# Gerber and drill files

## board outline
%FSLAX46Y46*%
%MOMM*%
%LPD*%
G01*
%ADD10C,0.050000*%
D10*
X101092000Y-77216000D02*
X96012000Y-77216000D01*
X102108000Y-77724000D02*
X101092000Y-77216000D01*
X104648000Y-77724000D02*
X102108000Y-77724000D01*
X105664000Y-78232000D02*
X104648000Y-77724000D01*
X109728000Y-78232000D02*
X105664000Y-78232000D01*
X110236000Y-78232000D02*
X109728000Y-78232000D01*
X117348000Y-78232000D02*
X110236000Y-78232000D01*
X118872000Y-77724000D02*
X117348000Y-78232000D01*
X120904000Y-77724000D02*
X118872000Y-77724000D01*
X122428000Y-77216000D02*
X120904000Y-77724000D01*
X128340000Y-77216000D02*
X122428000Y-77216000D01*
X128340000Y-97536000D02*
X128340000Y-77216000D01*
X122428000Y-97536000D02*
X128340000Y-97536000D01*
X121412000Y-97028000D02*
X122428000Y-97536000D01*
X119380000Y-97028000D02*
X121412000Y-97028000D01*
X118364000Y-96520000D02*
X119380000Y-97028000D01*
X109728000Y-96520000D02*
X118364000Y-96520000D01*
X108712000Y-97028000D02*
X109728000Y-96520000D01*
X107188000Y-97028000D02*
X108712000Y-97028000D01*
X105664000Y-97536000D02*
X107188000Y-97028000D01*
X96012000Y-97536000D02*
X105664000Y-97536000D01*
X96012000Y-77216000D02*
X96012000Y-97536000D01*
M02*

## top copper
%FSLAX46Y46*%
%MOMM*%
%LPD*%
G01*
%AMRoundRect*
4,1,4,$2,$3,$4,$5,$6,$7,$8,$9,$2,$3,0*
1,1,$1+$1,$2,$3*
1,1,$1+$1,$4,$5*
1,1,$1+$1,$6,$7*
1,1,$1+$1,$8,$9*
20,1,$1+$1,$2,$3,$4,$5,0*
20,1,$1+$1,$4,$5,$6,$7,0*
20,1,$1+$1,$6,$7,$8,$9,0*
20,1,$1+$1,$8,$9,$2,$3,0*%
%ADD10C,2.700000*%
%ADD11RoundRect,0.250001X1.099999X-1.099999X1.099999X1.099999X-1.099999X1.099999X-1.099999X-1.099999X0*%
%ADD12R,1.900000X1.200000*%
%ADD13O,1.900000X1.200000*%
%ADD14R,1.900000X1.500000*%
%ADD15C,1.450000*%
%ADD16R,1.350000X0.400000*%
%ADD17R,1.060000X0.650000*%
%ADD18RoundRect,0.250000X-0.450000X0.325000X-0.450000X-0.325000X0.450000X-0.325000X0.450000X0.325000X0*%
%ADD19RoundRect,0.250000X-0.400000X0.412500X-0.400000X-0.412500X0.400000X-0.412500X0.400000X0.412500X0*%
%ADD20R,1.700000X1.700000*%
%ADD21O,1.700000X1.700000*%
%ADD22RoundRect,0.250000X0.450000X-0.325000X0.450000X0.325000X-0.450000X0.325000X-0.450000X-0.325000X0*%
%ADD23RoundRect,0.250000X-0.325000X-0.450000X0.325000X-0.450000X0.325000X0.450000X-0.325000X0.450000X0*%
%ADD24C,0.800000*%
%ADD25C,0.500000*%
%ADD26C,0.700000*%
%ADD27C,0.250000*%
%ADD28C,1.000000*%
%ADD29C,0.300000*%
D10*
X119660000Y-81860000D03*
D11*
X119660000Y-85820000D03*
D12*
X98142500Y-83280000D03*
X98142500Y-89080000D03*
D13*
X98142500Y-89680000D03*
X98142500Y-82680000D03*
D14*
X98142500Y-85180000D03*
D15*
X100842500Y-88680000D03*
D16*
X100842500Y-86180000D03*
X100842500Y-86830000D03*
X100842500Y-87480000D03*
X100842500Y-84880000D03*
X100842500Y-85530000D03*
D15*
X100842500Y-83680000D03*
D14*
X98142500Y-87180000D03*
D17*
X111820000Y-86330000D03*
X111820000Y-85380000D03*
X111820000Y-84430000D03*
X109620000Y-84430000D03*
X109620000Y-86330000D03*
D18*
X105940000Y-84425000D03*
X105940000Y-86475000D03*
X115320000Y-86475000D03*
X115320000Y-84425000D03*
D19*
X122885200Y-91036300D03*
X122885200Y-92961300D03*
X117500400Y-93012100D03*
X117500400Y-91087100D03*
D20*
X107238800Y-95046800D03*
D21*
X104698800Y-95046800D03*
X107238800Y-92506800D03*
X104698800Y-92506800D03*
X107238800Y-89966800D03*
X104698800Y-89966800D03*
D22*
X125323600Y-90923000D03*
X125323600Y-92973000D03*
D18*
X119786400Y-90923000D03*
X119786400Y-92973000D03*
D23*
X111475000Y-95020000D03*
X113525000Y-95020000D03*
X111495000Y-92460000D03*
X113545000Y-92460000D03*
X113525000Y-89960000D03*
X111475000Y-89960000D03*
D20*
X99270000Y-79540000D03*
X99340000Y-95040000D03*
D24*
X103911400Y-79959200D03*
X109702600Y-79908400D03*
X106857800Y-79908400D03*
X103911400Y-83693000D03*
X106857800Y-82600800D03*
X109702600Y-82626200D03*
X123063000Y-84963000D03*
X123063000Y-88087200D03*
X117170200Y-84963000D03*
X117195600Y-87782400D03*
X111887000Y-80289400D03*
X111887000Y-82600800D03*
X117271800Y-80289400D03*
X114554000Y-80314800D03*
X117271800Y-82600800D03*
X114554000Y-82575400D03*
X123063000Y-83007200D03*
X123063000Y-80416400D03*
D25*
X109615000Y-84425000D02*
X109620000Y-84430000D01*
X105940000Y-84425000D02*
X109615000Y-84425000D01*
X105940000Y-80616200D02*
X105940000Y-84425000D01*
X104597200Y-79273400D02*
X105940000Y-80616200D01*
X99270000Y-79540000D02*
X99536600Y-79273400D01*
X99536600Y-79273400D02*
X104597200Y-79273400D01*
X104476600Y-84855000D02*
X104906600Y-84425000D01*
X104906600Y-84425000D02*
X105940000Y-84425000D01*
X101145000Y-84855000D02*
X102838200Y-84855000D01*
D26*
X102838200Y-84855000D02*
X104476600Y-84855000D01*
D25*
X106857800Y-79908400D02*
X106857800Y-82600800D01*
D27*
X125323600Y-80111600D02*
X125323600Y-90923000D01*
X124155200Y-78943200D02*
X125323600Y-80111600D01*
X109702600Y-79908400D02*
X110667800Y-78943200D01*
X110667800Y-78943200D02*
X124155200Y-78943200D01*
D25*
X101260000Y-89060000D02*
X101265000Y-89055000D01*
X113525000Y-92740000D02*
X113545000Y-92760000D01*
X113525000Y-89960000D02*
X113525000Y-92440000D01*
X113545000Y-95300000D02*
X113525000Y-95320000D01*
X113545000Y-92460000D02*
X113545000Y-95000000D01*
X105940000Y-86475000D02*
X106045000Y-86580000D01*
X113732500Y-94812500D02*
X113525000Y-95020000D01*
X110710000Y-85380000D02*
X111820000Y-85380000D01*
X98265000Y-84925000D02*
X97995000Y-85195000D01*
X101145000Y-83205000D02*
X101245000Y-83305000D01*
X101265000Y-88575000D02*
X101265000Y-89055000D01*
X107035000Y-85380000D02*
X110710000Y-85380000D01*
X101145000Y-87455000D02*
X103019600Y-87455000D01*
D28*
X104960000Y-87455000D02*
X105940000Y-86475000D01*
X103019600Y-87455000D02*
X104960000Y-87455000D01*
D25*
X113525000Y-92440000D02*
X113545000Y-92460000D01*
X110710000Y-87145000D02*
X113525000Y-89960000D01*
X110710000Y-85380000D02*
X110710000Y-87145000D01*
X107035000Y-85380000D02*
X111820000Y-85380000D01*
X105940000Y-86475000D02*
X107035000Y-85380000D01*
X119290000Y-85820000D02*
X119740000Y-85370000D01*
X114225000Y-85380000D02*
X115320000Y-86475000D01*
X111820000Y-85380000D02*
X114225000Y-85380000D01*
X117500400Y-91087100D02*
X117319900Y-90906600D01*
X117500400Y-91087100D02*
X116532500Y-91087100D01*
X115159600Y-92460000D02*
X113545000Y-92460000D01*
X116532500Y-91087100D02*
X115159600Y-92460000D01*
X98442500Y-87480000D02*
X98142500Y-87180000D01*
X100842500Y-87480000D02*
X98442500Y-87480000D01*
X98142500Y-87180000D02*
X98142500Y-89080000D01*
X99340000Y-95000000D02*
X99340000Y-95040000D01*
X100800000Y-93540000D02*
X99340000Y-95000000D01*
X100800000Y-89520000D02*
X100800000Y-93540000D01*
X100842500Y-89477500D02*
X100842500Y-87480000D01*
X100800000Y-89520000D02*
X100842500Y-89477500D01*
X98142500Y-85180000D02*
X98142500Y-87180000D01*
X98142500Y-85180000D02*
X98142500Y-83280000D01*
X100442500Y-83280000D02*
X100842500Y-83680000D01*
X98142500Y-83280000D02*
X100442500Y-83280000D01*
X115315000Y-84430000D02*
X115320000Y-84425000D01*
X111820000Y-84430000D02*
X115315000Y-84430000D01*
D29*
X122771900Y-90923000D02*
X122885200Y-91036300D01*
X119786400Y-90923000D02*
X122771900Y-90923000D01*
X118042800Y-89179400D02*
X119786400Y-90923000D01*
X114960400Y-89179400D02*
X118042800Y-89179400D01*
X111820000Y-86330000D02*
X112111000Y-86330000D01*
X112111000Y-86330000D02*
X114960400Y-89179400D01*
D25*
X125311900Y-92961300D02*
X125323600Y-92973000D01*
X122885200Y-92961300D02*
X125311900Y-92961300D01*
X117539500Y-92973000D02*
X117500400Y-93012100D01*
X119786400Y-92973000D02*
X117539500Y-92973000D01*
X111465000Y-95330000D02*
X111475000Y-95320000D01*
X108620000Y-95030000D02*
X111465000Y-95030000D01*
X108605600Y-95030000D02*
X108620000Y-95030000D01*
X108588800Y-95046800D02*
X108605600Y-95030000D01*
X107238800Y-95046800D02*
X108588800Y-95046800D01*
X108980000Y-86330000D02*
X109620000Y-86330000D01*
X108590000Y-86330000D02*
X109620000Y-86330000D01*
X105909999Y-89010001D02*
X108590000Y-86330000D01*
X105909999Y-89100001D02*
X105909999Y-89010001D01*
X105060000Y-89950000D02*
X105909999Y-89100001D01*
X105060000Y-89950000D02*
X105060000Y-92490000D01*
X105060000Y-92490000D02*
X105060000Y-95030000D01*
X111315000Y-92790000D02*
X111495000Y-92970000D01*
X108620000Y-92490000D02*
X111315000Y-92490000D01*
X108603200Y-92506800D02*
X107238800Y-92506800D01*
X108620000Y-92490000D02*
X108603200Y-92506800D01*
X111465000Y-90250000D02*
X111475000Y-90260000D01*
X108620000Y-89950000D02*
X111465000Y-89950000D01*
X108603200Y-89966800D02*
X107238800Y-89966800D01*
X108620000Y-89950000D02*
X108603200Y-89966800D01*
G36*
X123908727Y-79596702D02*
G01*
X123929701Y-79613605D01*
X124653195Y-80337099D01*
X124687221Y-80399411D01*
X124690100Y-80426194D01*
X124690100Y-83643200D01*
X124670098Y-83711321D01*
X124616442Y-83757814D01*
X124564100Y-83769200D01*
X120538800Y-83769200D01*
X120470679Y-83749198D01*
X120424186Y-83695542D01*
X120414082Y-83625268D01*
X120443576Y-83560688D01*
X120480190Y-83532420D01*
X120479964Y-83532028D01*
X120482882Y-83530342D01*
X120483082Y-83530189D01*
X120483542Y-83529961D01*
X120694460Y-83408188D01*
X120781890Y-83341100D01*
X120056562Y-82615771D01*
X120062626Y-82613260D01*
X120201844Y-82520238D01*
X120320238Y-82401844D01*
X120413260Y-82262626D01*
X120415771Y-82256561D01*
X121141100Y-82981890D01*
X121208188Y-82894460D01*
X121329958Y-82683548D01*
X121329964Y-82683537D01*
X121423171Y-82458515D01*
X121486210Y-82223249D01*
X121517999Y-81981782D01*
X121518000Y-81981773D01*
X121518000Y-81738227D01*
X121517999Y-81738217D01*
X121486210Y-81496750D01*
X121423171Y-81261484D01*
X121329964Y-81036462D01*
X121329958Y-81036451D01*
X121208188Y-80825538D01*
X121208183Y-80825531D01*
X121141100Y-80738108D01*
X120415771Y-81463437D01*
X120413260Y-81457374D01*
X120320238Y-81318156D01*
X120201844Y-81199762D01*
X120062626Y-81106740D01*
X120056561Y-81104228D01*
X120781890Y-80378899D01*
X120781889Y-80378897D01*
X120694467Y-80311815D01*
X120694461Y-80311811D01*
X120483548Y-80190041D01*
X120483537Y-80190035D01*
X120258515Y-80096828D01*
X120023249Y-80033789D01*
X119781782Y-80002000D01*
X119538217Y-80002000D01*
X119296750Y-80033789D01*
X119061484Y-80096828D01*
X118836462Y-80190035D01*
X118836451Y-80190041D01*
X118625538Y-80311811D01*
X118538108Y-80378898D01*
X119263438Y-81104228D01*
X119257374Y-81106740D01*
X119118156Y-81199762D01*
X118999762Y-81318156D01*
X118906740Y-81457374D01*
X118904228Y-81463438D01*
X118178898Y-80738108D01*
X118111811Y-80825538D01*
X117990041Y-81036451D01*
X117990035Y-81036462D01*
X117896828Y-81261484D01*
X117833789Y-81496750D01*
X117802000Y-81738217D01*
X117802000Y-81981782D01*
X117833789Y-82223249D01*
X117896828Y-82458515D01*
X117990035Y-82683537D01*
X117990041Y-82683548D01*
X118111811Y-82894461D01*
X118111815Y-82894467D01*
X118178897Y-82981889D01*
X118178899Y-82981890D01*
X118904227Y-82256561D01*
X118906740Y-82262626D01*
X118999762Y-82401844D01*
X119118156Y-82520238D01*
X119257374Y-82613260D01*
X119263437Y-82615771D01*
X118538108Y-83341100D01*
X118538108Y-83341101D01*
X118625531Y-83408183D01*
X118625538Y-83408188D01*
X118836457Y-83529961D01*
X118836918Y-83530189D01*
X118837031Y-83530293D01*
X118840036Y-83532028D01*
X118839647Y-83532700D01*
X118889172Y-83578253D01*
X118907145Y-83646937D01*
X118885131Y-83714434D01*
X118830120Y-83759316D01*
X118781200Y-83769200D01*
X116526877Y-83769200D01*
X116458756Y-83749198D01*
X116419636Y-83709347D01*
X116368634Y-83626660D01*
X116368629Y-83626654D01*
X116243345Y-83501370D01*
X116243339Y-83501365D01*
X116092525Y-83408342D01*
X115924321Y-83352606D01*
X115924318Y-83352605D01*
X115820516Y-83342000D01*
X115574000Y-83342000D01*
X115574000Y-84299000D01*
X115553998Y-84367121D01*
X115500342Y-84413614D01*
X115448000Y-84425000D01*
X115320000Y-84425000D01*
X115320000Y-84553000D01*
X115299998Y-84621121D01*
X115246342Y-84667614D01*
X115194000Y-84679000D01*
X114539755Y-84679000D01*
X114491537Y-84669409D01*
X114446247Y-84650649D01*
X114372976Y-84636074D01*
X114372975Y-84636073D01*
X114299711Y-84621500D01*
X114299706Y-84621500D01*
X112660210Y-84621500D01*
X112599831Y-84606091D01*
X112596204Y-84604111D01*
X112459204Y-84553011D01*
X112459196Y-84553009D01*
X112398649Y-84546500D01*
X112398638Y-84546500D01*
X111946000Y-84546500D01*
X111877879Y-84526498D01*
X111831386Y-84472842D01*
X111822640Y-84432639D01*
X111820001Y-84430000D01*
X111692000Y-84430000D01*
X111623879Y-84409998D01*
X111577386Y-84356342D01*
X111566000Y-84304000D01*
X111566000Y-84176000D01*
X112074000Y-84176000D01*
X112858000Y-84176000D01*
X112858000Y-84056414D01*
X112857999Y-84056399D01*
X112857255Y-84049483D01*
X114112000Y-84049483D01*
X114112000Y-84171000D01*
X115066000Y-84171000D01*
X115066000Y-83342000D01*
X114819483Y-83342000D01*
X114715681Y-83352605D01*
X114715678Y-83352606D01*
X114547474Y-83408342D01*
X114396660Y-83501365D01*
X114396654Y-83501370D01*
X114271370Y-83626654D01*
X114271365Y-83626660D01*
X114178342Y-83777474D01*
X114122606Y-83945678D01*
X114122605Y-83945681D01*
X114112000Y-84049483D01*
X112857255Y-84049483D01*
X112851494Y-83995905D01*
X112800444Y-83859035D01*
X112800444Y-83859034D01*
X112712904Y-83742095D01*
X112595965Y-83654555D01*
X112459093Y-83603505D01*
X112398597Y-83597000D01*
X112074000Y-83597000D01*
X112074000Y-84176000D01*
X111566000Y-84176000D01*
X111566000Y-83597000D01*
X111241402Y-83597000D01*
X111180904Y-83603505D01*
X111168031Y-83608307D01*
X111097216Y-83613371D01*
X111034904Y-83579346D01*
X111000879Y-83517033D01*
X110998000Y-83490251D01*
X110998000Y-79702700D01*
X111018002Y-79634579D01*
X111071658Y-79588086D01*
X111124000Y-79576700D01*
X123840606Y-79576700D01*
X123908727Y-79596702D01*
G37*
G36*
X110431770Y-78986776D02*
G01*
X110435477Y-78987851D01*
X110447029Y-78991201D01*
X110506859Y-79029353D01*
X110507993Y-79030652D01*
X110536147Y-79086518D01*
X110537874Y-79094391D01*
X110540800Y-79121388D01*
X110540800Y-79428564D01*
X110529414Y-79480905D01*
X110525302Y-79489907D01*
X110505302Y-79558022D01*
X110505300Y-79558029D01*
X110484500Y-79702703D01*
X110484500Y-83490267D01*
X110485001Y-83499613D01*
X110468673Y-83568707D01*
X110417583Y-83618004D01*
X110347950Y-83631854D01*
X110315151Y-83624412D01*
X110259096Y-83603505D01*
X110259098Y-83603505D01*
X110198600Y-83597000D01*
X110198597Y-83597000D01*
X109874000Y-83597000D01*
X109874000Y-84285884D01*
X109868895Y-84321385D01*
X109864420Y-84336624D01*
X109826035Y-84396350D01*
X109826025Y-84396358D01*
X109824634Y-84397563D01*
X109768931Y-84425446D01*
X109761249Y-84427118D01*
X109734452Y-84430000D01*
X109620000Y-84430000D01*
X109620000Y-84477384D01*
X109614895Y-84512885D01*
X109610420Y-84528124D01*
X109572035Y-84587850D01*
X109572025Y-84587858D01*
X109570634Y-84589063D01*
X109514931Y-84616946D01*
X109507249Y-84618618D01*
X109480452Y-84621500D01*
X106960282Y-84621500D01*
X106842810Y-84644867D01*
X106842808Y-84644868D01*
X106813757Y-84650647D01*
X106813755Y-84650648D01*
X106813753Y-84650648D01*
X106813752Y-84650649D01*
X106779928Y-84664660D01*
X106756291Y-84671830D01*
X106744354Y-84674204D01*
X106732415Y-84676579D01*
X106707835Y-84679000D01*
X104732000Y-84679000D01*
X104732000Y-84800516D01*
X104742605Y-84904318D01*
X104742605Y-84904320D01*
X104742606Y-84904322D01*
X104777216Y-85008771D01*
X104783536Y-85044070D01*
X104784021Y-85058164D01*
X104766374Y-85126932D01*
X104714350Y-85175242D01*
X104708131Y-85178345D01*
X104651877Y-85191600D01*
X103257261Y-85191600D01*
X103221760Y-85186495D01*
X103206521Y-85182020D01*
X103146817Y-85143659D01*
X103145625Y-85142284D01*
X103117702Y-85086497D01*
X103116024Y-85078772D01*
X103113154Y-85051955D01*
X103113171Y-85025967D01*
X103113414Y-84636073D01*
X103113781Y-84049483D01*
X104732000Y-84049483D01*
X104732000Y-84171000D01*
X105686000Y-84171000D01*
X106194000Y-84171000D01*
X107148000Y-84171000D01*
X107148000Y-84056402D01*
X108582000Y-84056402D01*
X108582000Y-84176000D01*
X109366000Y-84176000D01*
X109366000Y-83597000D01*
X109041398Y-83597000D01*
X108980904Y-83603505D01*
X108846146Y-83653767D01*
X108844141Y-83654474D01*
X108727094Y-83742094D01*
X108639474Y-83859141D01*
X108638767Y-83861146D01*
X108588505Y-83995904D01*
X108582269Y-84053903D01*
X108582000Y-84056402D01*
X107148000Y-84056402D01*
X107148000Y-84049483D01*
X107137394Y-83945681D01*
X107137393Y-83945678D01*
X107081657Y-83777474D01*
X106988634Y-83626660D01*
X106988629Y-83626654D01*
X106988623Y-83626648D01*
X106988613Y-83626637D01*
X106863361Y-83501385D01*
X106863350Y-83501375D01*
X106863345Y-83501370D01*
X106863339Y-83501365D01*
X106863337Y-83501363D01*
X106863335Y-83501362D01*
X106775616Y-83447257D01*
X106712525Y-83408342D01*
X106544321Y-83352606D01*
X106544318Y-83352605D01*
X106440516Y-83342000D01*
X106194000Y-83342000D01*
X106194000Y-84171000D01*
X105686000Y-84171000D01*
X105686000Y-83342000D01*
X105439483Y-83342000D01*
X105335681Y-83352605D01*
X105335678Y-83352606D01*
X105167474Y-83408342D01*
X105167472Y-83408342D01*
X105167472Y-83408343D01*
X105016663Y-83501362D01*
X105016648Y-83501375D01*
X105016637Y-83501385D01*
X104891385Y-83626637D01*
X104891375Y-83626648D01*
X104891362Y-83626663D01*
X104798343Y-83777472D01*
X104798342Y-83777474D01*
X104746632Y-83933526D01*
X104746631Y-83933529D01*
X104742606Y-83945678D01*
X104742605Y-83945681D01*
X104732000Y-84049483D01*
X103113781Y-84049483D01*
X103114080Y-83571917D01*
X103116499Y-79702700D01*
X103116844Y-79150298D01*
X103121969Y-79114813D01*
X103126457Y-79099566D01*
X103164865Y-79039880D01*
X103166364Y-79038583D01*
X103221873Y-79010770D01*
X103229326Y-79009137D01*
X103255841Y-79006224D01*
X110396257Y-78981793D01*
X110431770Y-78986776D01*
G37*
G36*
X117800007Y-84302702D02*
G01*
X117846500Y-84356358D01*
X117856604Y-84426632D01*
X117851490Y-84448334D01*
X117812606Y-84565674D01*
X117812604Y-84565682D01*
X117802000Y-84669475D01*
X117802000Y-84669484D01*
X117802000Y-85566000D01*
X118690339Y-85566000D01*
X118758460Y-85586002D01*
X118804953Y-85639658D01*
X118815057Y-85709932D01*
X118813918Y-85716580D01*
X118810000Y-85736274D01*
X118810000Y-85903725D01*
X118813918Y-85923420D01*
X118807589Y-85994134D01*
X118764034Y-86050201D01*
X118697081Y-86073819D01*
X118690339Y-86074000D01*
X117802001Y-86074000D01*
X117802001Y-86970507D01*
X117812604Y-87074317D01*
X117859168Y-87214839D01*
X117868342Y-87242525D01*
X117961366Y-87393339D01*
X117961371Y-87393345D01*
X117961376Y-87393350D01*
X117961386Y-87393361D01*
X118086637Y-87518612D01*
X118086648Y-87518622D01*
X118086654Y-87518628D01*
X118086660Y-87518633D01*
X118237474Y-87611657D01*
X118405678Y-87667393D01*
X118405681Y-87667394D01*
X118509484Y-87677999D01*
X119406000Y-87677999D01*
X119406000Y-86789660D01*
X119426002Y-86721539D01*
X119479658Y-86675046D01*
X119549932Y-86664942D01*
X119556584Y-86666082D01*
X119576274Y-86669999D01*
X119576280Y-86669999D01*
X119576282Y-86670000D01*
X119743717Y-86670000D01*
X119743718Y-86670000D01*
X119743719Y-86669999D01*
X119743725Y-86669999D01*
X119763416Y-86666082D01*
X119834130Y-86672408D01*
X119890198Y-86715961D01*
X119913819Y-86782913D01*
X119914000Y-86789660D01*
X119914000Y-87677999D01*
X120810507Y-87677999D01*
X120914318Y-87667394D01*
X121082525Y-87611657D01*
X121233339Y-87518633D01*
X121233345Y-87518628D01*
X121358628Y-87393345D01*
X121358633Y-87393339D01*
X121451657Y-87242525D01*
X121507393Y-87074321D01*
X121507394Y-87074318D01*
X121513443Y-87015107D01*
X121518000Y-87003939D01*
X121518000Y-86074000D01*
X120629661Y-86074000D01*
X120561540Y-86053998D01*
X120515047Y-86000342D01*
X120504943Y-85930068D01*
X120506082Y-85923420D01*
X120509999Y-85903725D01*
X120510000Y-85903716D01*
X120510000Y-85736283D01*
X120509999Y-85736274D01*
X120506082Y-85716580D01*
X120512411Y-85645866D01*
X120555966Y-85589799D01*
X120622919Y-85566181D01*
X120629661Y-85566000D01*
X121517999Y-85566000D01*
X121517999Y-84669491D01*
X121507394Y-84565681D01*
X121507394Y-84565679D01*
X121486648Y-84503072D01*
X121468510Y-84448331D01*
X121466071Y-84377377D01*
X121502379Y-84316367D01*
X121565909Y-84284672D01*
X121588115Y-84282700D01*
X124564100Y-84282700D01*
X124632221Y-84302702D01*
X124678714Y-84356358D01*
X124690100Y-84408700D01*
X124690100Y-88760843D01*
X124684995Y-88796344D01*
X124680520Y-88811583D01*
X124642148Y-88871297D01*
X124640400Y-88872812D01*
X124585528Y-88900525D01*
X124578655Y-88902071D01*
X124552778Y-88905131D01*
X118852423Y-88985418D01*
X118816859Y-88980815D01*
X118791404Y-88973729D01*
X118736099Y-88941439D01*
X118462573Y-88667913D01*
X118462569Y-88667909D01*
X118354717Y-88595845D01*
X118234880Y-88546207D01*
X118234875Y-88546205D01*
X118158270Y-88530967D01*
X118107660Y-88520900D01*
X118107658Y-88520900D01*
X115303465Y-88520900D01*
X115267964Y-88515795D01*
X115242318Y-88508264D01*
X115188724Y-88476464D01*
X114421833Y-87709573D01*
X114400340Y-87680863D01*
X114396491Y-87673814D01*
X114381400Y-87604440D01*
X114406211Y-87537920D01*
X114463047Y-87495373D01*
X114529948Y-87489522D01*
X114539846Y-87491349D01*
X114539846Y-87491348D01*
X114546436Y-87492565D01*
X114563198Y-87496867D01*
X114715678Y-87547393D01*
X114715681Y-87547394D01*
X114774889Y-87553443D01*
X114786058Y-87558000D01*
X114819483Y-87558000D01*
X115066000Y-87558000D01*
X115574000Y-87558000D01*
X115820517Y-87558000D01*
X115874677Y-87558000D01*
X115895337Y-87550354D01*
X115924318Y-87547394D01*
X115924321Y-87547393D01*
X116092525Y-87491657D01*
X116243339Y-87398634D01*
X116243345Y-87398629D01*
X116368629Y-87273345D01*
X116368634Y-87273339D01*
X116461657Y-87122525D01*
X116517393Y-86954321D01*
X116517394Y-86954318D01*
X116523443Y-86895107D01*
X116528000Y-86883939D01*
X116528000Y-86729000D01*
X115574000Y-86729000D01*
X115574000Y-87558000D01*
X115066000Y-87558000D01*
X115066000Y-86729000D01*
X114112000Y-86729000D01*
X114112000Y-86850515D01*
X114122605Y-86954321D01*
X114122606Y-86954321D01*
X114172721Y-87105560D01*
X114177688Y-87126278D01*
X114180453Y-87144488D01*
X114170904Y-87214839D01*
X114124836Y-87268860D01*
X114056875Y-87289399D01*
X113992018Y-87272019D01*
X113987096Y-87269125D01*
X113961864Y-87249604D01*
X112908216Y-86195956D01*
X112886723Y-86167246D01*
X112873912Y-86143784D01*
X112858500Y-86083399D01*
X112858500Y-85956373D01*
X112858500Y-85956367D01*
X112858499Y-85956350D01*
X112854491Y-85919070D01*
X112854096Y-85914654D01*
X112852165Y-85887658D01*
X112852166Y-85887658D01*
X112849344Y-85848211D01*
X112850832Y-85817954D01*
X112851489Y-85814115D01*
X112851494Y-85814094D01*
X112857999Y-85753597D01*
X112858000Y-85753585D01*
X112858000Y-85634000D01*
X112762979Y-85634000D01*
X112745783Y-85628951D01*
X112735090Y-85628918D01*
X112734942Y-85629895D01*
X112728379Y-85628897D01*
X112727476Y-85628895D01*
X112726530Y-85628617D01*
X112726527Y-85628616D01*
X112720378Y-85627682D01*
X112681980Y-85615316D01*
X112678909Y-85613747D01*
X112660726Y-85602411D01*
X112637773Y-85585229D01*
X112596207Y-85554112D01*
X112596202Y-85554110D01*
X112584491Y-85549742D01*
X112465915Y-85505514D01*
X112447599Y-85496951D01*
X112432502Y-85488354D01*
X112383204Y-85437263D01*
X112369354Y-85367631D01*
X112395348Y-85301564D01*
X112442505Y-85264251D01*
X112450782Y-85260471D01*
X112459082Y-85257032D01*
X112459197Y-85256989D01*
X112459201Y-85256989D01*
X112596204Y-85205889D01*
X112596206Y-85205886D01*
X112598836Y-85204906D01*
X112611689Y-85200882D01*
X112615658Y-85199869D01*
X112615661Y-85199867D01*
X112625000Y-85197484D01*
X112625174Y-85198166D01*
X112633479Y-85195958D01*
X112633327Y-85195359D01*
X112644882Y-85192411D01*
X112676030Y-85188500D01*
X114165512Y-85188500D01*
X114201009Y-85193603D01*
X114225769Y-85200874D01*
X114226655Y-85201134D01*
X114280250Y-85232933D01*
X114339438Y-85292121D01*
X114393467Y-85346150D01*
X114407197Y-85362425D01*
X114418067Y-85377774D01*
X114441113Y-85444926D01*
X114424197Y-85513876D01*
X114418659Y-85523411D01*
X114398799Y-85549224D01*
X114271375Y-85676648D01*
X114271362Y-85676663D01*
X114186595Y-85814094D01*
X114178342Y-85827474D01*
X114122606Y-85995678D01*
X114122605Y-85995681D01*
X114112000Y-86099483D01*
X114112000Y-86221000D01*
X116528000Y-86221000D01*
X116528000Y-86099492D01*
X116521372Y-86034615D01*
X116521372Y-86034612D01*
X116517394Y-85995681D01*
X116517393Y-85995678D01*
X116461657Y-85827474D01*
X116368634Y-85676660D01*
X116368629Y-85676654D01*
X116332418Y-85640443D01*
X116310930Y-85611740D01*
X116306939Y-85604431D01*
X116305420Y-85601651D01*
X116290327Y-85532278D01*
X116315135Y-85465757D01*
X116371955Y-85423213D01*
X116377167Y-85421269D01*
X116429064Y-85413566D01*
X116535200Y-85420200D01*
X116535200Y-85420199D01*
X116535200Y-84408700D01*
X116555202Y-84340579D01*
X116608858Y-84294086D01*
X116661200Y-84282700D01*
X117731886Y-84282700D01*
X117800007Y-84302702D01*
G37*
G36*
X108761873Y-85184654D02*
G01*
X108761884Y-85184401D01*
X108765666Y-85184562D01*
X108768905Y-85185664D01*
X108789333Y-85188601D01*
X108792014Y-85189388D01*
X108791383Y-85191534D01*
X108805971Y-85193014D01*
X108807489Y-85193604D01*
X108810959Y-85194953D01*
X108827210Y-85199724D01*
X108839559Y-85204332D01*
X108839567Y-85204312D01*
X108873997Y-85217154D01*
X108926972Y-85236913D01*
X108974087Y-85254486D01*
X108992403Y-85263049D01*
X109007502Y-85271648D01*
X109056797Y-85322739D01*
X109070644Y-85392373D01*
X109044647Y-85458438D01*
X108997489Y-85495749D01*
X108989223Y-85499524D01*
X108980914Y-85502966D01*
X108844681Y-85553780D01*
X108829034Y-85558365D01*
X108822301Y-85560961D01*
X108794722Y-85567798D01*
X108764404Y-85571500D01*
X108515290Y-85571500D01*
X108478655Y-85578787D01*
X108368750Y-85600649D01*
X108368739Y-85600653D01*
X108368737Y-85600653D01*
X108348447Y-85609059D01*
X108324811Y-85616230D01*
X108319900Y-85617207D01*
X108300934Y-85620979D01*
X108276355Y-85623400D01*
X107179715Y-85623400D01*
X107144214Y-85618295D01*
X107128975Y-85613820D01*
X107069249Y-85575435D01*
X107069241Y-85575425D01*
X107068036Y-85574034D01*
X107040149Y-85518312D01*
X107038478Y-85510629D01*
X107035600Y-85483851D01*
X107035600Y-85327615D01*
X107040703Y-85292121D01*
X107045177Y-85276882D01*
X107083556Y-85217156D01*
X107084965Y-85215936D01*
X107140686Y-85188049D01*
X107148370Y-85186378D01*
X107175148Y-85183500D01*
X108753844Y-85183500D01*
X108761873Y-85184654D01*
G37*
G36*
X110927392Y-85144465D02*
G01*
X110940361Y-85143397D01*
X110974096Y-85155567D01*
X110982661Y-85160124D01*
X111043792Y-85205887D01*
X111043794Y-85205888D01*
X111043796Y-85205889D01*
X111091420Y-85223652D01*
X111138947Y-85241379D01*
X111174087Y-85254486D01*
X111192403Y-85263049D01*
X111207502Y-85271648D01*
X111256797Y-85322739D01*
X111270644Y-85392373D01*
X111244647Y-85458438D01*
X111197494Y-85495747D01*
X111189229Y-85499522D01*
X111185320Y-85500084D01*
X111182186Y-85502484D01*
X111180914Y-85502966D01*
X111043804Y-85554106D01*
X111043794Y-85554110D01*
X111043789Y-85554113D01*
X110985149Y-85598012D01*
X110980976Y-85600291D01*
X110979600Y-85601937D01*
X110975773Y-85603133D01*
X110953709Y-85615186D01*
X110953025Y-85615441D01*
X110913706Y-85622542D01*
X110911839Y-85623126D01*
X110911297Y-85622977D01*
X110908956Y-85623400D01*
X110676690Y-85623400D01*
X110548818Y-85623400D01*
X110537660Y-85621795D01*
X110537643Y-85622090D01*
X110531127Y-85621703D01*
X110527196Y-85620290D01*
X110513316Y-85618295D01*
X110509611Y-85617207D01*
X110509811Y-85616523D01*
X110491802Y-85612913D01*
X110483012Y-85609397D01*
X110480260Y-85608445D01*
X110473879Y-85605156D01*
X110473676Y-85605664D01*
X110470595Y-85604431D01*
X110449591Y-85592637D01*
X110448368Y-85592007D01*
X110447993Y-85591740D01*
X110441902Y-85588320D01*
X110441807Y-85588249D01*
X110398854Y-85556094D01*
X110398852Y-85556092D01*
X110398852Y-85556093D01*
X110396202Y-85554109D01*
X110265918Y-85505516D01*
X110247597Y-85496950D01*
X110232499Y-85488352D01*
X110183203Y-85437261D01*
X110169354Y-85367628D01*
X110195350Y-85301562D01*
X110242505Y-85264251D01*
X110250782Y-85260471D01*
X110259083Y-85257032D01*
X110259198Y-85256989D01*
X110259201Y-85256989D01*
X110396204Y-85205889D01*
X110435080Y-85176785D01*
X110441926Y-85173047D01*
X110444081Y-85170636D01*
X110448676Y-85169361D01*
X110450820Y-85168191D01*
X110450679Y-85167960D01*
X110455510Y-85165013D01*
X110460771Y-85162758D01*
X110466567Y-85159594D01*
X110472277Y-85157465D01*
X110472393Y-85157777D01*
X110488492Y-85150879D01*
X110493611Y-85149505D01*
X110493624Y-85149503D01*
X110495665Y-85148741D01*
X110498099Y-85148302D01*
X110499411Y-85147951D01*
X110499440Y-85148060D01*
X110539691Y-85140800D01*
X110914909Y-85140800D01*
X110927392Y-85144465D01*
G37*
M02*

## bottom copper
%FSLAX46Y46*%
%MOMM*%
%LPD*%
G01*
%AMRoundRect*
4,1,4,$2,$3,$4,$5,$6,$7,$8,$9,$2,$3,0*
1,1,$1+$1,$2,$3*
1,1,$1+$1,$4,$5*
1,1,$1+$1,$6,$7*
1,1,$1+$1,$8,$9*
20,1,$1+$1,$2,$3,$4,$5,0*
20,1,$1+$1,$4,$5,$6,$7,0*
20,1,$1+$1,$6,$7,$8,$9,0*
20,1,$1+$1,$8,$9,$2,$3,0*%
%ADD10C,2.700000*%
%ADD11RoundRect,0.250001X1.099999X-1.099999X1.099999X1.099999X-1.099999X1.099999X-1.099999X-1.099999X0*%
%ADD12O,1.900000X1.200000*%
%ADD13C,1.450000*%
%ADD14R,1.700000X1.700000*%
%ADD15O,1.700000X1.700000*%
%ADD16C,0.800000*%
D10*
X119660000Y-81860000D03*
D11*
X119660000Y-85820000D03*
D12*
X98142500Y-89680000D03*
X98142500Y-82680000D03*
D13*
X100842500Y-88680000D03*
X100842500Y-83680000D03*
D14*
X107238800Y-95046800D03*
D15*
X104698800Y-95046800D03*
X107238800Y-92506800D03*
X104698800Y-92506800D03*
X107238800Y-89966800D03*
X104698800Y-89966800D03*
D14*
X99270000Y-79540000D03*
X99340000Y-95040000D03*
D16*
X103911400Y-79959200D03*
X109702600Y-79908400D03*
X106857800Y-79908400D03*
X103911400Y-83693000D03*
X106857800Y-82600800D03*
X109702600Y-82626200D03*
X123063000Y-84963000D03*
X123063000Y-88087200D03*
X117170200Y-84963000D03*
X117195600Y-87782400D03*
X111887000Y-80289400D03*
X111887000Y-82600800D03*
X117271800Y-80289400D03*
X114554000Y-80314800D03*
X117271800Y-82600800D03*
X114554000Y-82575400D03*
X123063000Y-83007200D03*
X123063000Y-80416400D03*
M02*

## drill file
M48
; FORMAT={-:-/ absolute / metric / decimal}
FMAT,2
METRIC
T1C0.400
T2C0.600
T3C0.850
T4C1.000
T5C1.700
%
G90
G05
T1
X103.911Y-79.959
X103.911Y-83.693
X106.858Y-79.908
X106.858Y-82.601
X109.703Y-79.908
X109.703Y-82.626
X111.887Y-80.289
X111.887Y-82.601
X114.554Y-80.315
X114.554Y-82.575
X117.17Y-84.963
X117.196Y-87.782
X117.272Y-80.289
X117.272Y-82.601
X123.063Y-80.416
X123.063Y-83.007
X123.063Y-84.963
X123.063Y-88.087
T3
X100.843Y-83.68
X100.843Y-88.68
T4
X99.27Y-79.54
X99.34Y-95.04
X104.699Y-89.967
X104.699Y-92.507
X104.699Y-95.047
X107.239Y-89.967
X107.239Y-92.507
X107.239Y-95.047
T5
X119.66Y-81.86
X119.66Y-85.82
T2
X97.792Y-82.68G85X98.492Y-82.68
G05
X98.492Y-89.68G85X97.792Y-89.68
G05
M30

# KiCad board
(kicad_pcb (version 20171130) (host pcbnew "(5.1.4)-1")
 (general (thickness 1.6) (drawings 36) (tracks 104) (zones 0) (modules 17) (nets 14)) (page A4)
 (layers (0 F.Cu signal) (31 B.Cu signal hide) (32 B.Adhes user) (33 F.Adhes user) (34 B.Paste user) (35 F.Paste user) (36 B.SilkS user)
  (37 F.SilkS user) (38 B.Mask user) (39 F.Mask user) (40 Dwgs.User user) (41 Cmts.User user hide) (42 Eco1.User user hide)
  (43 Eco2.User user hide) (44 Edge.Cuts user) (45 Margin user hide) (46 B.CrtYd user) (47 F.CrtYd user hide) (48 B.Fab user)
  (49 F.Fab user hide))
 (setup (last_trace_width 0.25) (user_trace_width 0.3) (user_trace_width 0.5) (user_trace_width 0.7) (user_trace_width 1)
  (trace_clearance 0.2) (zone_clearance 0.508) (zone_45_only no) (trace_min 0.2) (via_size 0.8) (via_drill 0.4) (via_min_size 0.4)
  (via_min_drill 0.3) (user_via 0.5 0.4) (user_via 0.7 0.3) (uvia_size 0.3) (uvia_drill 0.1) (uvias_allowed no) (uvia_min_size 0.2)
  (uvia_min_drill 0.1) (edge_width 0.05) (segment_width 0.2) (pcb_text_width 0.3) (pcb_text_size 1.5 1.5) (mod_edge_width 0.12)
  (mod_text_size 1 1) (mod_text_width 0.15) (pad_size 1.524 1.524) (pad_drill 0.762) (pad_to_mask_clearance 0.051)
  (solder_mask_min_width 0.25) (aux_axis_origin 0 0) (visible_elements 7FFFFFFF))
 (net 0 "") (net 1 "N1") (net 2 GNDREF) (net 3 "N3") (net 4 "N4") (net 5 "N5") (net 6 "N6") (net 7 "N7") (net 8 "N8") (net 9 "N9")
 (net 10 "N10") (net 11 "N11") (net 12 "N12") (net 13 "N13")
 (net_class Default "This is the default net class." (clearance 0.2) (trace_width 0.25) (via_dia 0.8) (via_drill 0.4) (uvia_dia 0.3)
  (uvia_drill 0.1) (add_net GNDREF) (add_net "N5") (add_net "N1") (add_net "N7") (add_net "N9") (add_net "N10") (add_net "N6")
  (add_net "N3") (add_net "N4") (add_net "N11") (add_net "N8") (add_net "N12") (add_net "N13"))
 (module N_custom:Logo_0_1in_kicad (layer F.Cu) (at 108.3 81.51)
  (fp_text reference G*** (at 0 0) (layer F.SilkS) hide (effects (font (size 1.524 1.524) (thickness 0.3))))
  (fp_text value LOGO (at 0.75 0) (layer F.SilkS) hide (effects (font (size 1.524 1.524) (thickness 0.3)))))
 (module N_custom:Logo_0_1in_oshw (layer F.Cu) (at 115.92 81.36)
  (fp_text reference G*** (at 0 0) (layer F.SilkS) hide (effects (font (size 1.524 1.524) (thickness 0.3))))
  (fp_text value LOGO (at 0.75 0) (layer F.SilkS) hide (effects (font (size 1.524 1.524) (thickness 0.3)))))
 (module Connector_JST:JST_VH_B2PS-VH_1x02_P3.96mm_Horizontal (layer F.Cu) (at 119.66 85.82 90)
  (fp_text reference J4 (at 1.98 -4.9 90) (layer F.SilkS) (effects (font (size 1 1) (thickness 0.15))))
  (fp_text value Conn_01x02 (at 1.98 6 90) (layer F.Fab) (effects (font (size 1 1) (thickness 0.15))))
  (pad 2 thru_hole circle (at 3.96 0 90) (size 2.7 2.7) (drill 1.7) (layers *.Cu *.Mask) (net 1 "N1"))
  (pad 1 thru_hole roundrect (at 0 0 90) (size 2.7 2.7) (drill 1.7) (layers *.Cu *.Mask) (roundrect_rratio 0.09259299999999999)
   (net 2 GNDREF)))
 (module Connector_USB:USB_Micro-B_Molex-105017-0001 (layer F.Cu) (at 99.38 86.18 270)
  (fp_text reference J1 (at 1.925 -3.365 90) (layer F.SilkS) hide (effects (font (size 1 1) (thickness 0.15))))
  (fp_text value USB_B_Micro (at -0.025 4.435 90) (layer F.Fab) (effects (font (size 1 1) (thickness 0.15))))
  (pad 6 smd rect (at -2.9 1.2375 270) (size 1.2 1.9) (layers F.Cu F.Mask) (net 2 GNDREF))
  (pad 6 smd rect (at 2.9 1.2375 270) (size 1.2 1.9) (layers F.Cu F.Mask) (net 2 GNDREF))
  (pad 6 thru_hole oval (at 3.5 1.2375 270) (size 1.2 1.9) (drill oval 0.6 1.3) (layers *.Cu *.Mask) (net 2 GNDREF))
  (pad 6 thru_hole oval (at -3.5 1.2375 90) (size 1.2 1.9) (drill oval 0.6 1.3) (layers *.Cu *.Mask) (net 2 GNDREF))
  (pad 6 smd rect (at -1 1.2375 270) (size 1.5 1.9) (layers F.Cu F.Paste F.Mask) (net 2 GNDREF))
  (pad 6 thru_hole circle (at 2.5 -1.4625 270) (size 1.45 1.45) (drill 0.85) (layers *.Cu *.Mask) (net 2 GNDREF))
  (pad 3 smd rect (at 0 -1.4625 270) (size 0.4 1.35) (layers F.Cu F.Paste F.Mask) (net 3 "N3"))
  (pad 4 smd rect (at 0.65 -1.4625 270) (size 0.4 1.35) (layers F.Cu F.Paste F.Mask) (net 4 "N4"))
  (pad 5 smd rect (at 1.3 -1.4625 270) (size 0.4 1.35) (layers F.Cu F.Paste F.Mask) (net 2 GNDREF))
  (pad 1 smd rect (at -1.3 -1.4625 270) (size 0.4 1.35) (layers F.Cu F.Paste F.Mask) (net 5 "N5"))
  (pad 2 smd rect (at -0.65 -1.4625 270) (size 0.4 1.35) (layers F.Cu F.Paste F.Mask) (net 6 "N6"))
  (pad 6 thru_hole circle (at -2.5 -1.4625 270) (size 1.45 1.45) (drill 0.85) (layers *.Cu *.Mask) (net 2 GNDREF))
  (pad 6 smd rect (at 1 1.2375 270) (size 1.5 1.9) (layers F.Cu F.Paste F.Mask) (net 2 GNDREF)))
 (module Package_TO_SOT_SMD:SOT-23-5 (layer F.Cu) (at 110.72 85.38 180)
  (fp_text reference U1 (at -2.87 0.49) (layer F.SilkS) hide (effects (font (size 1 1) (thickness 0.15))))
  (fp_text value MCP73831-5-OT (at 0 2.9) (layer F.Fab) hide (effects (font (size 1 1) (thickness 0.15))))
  (pad 1 smd rect (at -1.1 -0.95 180) (size 1.06 0.65) (layers F.Cu F.Paste F.Mask) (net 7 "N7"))
  (pad 2 smd rect (at -1.1 0 180) (size 1.06 0.65) (layers F.Cu F.Paste F.Mask) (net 2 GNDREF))
  (pad 3 smd rect (at -1.1 0.95 180) (size 1.06 0.65) (layers F.Cu F.Paste F.Mask) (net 1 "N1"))
  (pad 4 smd rect (at 1.1 0.95 180) (size 1.06 0.65) (layers F.Cu F.Paste F.Mask) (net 5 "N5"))
  (pad 5 smd rect (at 1.1 -0.95 180) (size 1.06 0.65) (layers F.Cu F.Paste F.Mask) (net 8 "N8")))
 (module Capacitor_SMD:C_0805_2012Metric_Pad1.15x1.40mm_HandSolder (layer F.Cu) (at 105.94 85.45 270)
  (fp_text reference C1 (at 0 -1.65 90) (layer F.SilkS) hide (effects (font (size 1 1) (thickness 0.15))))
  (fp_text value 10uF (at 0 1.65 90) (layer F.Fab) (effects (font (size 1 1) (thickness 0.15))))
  (pad 1 smd roundrect (at -1.025 0 270) (size 1.15 1.4) (layers F.Cu F.Paste F.Mask) (roundrect_rratio 0.217391) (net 5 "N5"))
  (pad 2 smd roundrect (at 1.025 0 270) (size 1.15 1.4) (layers F.Cu F.Paste F.Mask) (roundrect_rratio 0.217391) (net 2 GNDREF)))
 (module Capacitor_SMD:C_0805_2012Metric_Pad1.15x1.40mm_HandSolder (layer F.Cu) (at 115.32 85.45 270)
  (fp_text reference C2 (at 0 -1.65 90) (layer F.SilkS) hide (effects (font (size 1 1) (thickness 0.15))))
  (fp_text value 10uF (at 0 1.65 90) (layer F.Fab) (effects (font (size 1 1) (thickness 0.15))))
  (pad 2 smd roundrect (at 1.025 0 270) (size 1.15 1.4) (layers F.Cu F.Paste F.Mask) (roundrect_rratio 0.217391) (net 2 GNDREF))
  (pad 1 smd roundrect (at -1.025 0 270) (size 1.15 1.4) (layers F.Cu F.Paste F.Mask) (roundrect_rratio 0.217391) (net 1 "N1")))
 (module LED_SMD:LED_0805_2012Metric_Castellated (layer F.Cu) (at 122.8852 91.9988 270)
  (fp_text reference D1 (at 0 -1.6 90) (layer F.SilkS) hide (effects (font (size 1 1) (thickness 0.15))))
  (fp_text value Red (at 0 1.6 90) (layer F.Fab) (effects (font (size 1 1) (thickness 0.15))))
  (pad 1 smd roundrect (at -0.9625 0 270) (size 1.325 1.3) (layers F.Cu F.Paste F.Mask) (roundrect_rratio 0.192308) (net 7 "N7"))
  (pad 2 smd roundrect (at 0.9625 0 270) (size 1.325 1.3) (layers F.Cu F.Paste F.Mask) (roundrect_rratio 0.192308) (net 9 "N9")))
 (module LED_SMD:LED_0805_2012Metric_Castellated (layer F.Cu) (at 117.5004 92.0496 270)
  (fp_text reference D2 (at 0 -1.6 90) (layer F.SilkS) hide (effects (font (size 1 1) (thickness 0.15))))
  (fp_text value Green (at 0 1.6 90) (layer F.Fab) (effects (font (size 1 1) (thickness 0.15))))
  (pad 2 smd roundrect (at 0.9625 0 270) (size 1.325 1.3) (layers F.Cu F.Paste F.Mask) (roundrect_rratio 0.192308) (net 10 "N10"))
  (pad 1 smd roundrect (at -0.9625 0 270) (size 1.325 1.3) (layers F.Cu F.Paste F.Mask) (roundrect_rratio 0.192308) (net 2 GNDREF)))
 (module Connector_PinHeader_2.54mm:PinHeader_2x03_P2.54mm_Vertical (layer F.Cu) (at 107.2388 95.0468 180)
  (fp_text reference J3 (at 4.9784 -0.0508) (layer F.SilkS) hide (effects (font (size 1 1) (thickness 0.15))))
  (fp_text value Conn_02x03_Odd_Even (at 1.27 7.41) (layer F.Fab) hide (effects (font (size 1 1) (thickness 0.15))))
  (pad 1 thru_hole rect (at 0 0 180) (size 1.7 1.7) (drill 1) (layers *.Cu *.Mask) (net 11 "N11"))
  (pad 2 thru_hole oval (at 2.54 0 180) (size 1.7 1.7) (drill 1) (layers *.Cu *.Mask) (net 8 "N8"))
  (pad 3 thru_hole oval (at 0 2.54 180) (size 1.7 1.7) (drill 1) (layers *.Cu *.Mask) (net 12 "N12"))
  (pad 4 thru_hole oval (at 2.54 2.54 180) (size 1.7 1.7) (drill 1) (layers *.Cu *.Mask) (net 8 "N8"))
  (pad 5 thru_hole oval (at 0 5.08 180) (size 1.7 1.7) (drill 1) (layers *.Cu *.Mask) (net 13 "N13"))
  (pad 6 thru_hole oval (at 2.54 5.08 180) (size 1.7 1.7) (drill 1) (layers *.Cu *.Mask) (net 8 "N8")))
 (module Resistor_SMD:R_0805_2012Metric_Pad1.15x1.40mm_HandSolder (layer F.Cu) (at 125.3236 91.948 90)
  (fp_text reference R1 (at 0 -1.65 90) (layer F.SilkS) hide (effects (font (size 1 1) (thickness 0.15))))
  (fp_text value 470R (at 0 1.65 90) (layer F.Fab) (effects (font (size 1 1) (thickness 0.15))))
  (pad 2 smd roundrect (at 1.025 0 90) (size 1.15 1.4) (layers F.Cu F.Paste F.Mask) (roundrect_rratio 0.217391) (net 5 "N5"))
  (pad 1 smd roundrect (at -1.025 0 90) (size 1.15 1.4) (layers F.Cu F.Paste F.Mask) (roundrect_rratio 0.217391) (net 9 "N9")))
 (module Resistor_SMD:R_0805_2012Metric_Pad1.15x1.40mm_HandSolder (layer F.Cu) (at 119.7864 91.948 270)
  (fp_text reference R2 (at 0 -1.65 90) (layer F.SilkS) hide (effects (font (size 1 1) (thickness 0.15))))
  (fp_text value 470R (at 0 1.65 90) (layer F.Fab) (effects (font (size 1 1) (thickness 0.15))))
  (pad 1 smd roundrect (at -1.025 0 270) (size 1.15 1.4) (layers F.Cu F.Paste F.Mask) (roundrect_rratio 0.217391) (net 7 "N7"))
  (pad 2 smd roundrect (at 1.025 0 270) (size 1.15 1.4) (layers F.Cu F.Paste F.Mask) (roundrect_rratio 0.217391) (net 10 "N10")))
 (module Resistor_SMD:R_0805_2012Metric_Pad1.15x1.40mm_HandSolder (layer F.Cu) (at 112.5 95.02)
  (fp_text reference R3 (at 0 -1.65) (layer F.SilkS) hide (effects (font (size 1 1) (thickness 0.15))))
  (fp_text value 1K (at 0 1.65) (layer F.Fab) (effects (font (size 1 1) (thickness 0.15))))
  (pad 1 smd roundrect (at -1.025 0) (size 1.15 1.4) (layers F.Cu F.Paste F.Mask) (roundrect_rratio 0.217391) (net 11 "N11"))
  (pad 2 smd roundrect (at 1.025 0) (size 1.15 1.4) (layers F.Cu F.Paste F.Mask) (roundrect_rratio 0.217391) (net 2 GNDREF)))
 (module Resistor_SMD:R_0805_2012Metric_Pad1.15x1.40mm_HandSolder (layer F.Cu) (at 112.52 92.46)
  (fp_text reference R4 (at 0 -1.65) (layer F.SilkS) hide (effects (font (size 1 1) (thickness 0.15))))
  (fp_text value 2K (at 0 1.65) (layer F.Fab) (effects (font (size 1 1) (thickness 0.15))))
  (pad 1 smd roundrect (at -1.025 0) (size 1.15 1.4) (layers F.Cu F.Paste F.Mask) (roundrect_rratio 0.217391) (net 12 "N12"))
  (pad 2 smd roundrect (at 1.025 0) (size 1.15 1.4) (layers F.Cu F.Paste F.Mask) (roundrect_rratio 0.217391) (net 2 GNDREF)))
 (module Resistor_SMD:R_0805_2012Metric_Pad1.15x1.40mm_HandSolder (layer F.Cu) (at 112.5 89.96)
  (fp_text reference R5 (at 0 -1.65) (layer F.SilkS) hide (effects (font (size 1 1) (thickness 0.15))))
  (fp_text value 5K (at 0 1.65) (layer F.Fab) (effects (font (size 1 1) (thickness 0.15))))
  (pad 2 smd roundrect (at 1.025 0) (size 1.15 1.4) (layers F.Cu F.Paste F.Mask) (roundrect_rratio 0.217391) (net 2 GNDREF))
  (pad 1 smd roundrect (at -1.025 0) (size 1.15 1.4) (layers F.Cu F.Paste F.Mask) (roundrect_rratio 0.217391) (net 13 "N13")))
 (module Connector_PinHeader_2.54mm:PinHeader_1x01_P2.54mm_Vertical (layer F.Cu) (at 99.27 79.54)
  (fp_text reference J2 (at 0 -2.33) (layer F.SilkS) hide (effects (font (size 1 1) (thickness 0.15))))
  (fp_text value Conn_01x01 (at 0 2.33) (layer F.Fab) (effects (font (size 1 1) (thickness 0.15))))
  (pad 1 thru_hole rect (at 0 0) (size 1.7 1.7) (drill 1) (layers *.Cu *.Mask) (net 5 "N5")))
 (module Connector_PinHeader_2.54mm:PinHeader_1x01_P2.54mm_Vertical (layer F.Cu) (at 99.34 95.04)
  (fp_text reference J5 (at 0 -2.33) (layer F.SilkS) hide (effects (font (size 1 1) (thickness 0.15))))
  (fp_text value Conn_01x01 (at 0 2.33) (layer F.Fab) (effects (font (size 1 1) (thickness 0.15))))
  (pad 1 thru_hole rect (at 0 0) (size 1.7 1.7) (drill 1) (layers *.Cu *.Mask) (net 2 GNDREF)))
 (gr_line (start 101.092 77.216) (end 96.012 77.216) (layer Edge.Cuts) (width 0.05))
 (gr_line (start 102.108 77.724) (end 101.092 77.216) (layer Edge.Cuts) (width 0.05))
 (gr_line (start 104.648 77.724) (end 102.108 77.724) (layer Edge.Cuts) (width 0.05))
 (gr_line (start 105.664 78.232) (end 104.648 77.724) (layer Edge.Cuts) (width 0.05))
 (gr_line (start 109.728 78.232) (end 105.664 78.232) (layer Edge.Cuts) (width 0.05))
 (gr_line (start 110.236 78.232) (end 109.728 78.232) (layer Edge.Cuts) (width 0.05))
 (gr_line (start 117.348 78.232) (end 110.236 78.232) (layer Edge.Cuts) (width 0.05))
 (gr_line (start 118.872 77.724) (end 117.348 78.232) (layer Edge.Cuts) (width 0.05))
 (gr_line (start 120.904 77.724) (end 118.872 77.724) (layer Edge.Cuts) (width 0.05))
 (gr_line (start 122.428 77.216) (end 120.904 77.724) (layer Edge.Cuts) (width 0.05))
 (gr_line (start 128.34 77.216) (end 122.428 77.216) (layer Edge.Cuts) (width 0.05))
 (gr_line (start 128.34 97.536) (end 128.34 77.216) (layer Edge.Cuts) (width 0.05))
 (gr_line (start 122.428 97.536) (end 128.34 97.536) (layer Edge.Cuts) (width 0.05))
 (gr_line (start 121.412 97.028) (end 122.428 97.536) (layer Edge.Cuts) (width 0.05))
 (gr_line (start 119.38 97.028) (end 121.412 97.028) (layer Edge.Cuts) (width 0.05))
 (gr_line (start 118.364 96.52) (end 119.38 97.028) (layer Edge.Cuts) (width 0.05))
 (gr_line (start 109.728 96.52) (end 118.364 96.52) (layer Edge.Cuts) (width 0.05))
 (gr_line (start 108.712 97.028) (end 109.728 96.52) (layer Edge.Cuts) (width 0.05))
 (gr_line (start 107.188 97.028) (end 108.712 97.028) (layer Edge.Cuts) (width 0.05))
 (gr_line (start 105.664 97.536) (end 107.188 97.028) (layer Edge.Cuts) (width 0.05))
 (gr_line (start 96.012 97.536) (end 105.664 97.536) (layer Edge.Cuts) (width 0.05))
 (gr_line (start 96.012 77.216) (end 96.012 97.536) (layer Edge.Cuts) (width 0.05))
 (segment (start 109.615 84.425) (end 109.62 84.43) (width 0.5) (layer F.Cu) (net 5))
 (segment (start 105.94 84.425) (end 109.615 84.425) (width 0.5) (layer F.Cu) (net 5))
 (segment (start 105.94 80.6162) (end 105.94 84.425) (width 0.5) (layer F.Cu) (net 5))
 (segment (start 104.5972 79.2734) (end 105.94 80.6162) (width 0.5) (layer F.Cu) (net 5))
 (segment (start 99.27 79.54) (end 99.5366 79.2734) (width 0.5) (layer F.Cu) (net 5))
 (segment (start 99.5366 79.2734) (end 104.5972 79.2734) (width 0.5) (layer F.Cu) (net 5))
 (segment (start 104.4766 84.855) (end 104.9066 84.425) (width 0.5) (layer F.Cu) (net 5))
 (segment (start 104.9066 84.425) (end 105.94 84.425) (width 0.5) (layer F.Cu) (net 5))
 (segment (start 101.145 84.855) (end 102.8382 84.855) (width 0.5) (layer F.Cu) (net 5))
 (segment (start 102.8382 84.855) (end 104.4766 84.855) (width 0.7) (layer F.Cu) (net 5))
 (via (at 103.9114 79.9592) (size 0.8) (drill 0.4) (layers F.Cu B.Cu) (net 5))
 (via (at 109.7026 79.9084) (size 0.8) (drill 0.4) (layers F.Cu B.Cu) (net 5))
 (via (at 106.8578 79.9084) (size 0.8) (drill 0.4) (layers F.Cu B.Cu) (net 5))
 (via (at 103.9114 83.693) (size 0.8) (drill 0.4) (layers F.Cu B.Cu) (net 5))
 (via (at 106.8578 82.6008) (size 0.8) (drill 0.4) (layers F.Cu B.Cu) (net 5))
 (segment (start 106.8578 79.9084) (end 106.8578 82.6008) (width 0.5) (layer F.Cu) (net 5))
 (via (at 109.7026 82.6262) (size 0.8) (drill 0.4) (layers F.Cu B.Cu) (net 5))
 (segment (start 125.3236 80.1116) (end 125.3236 90.923) (width 0.25) (layer F.Cu) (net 5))
 (segment (start 124.1552 78.9432) (end 125.3236 80.1116) (width 0.25) (layer F.Cu) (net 5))
 (segment (start 109.7026 79.9084) (end 110.6678 78.9432) (width 0.25) (layer F.Cu) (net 5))
 (segment (start 110.6678 78.9432) (end 124.1552 78.9432) (width 0.25) (layer F.Cu) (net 5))
 (segment (start 101.26 89.06) (end 101.265 89.055) (width 0.5) (layer F.Cu) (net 2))
 (segment (start 113.525 92.74) (end 113.545 92.76) (width 0.5) (layer F.Cu) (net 2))
 (segment (start 113.525 89.96) (end 113.525 92.44) (width 0.5) (layer F.Cu) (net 2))
 (segment (start 113.545 95.3) (end 113.525 95.32) (width 0.5) (layer F.Cu) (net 2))
 (segment (start 113.545 92.46) (end 113.545 95) (width 0.5) (layer F.Cu) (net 2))
 (segment (start 105.94 86.475) (end 106.045 86.58) (width 0.5) (layer F.Cu) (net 2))
 (segment (start 113.7325 94.8125) (end 113.525 95.02) (width 0.5) (layer F.Cu) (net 2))
 (segment (start 110.71 85.38) (end 111.82 85.38) (width 0.5) (layer F.Cu) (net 2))
 (segment (start 98.265 84.925) (end 97.995 85.195) (width 0.5) (layer F.Cu) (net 2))
 (segment (start 101.145 83.205) (end 101.245 83.305) (width 0.5) (layer F.Cu) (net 2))
 (segment (start 101.265 88.575) (end 101.265 89.055) (width 0.5) (layer F.Cu) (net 2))
 (segment (start 107.035 85.38) (end 110.71 85.38) (width 0.5) (layer F.Cu) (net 2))
 (segment (start 101.145 87.455) (end 103.0196 87.455) (width 0.5) (layer F.Cu) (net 2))
 (segment (start 104.96 87.455) (end 105.94 86.475) (width 1) (layer F.Cu) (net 2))
 (segment (start 103.0196 87.455) (end 104.96 87.455) (width 1) (layer F.Cu) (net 2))
 (segment (start 113.525 92.44) (end 113.545 92.46) (width 0.5) (layer F.Cu) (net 2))
 (segment (start 110.71 87.145) (end 113.525 89.96) (width 0.5) (layer F.Cu) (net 2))
 (segment (start 110.71 85.38) (end 110.71 87.145) (width 0.5) (layer F.Cu) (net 2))
 (segment (start 107.035 85.38) (end 111.82 85.38) (width 0.5) (layer F.Cu) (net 2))
 (segment (start 105.94 86.475) (end 107.035 85.38) (width 0.5) (layer F.Cu) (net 2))
 (segment (start 119.29 85.82) (end 119.74 85.37) (width 0.5) (layer F.Cu) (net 2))
 (via (at 123.063 84.963) (size 0.8) (drill 0.4) (layers F.Cu B.Cu) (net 2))
 (via (at 123.063 88.0872) (size 0.8) (drill 0.4) (layers F.Cu B.Cu) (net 2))
 (via (at 117.1702 84.963) (size 0.8) (drill 0.4) (layers F.Cu B.Cu) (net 2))
 (via (at 117.1956 87.7824) (size 0.8) (drill 0.4) (layers F.Cu B.Cu) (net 2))
 (segment (start 114.225 85.38) (end 115.32 86.475) (width 0.5) (layer F.Cu) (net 2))
 (segment (start 111.82 85.38) (end 114.225 85.38) (width 0.5) (layer F.Cu) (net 2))
 (segment (start 117.5004 91.0871) (end 117.3199 90.9066) (width 0.5) (layer F.Cu) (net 2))
 (segment (start 117.5004 91.0871) (end 116.5325 91.0871) (width 0.5) (layer F.Cu) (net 2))
 (segment (start 115.1596 92.46) (end 113.545 92.46) (width 0.5) (layer F.Cu) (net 2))
 (segment (start 116.5325 91.0871) (end 115.1596 92.46) (width 0.5) (layer F.Cu) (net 2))
 (segment (start 98.4425 87.48) (end 98.1425 87.18) (width 0.5) (layer F.Cu) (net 2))
 (segment (start 100.8425 87.48) (end 98.4425 87.48) (width 0.5) (layer F.Cu) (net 2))
 (segment (start 98.1425 87.18) (end 98.1425 89.08) (width 0.5) (layer F.Cu) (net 2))
 (segment (start 99.34 95) (end 99.34 95.04) (width 0.5) (layer F.Cu) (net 2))
 (segment (start 100.8 93.54) (end 99.34 95) (width 0.5) (layer F.Cu) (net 2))
 (segment (start 100.8 89.52) (end 100.8 93.54) (width 0.5) (layer F.Cu) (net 2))
 (segment (start 100.8425 89.4775) (end 100.8425 87.48) (width 0.5) (layer F.Cu) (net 2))
 (segment (start 100.8 89.52) (end 100.8425 89.4775) (width 0.5) (layer F.Cu) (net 2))
 (segment (start 98.1425 85.18) (end 98.1425 87.18) (width 0.5) (layer F.Cu) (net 2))
 (segment (start 98.1425 85.18) (end 98.1425 83.28) (width 0.5) (layer F.Cu) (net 2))
 (segment (start 100.4425 83.28) (end 100.8425 83.68) (width 0.5) (layer F.Cu) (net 2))
 (segment (start 98.1425 83.28) (end 100.4425 83.28) (width 0.5) (layer F.Cu) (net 2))
 (segment (start 115.315 84.43) (end 115.32 84.425) (width 0.5) (layer F.Cu) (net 1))
 (segment (start 111.82 84.43) (end 115.315 84.43) (width 0.5) (layer F.Cu) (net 1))
 (via (at 111.887 80.2894) (size 0.8) (drill 0.4) (layers F.Cu B.Cu) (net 1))
 (via (at 111.887 82.6008) (size 0.8) (drill 0.4) (layers F.Cu B.Cu) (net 1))
 (via (at 117.2718 80.2894) (size 0.8) (drill 0.4) (layers F.Cu B.Cu) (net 1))
 (via (at 114.554 80.3148) (size 0.8) (drill 0.4) (layers F.Cu B.Cu) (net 1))
 (via (at 117.2718 82.6008) (size 0.8) (drill 0.4) (layers F.Cu B.Cu) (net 1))
 (via (at 114.554 82.5754) (size 0.8) (drill 0.4) (layers F.Cu B.Cu) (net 1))
 (via (at 123.063 83.0072) (size 0.8) (drill 0.4) (layers F.Cu B.Cu) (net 1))
 (via (at 123.063 80.4164) (size 0.8) (drill 0.4) (layers F.Cu B.Cu) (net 1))
 (segment (start 122.7719 90.923) (end 122.8852 91.0363) (width 0.3) (layer F.Cu) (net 7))
 (segment (start 119.7864 90.923) (end 122.7719 90.923) (width 0.3) (layer F.Cu) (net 7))
 (segment (start 118.0428 89.1794) (end 119.7864 90.923) (width 0.3) (layer F.Cu) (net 7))
 (segment (start 114.9604 89.1794) (end 118.0428 89.1794) (width 0.3) (layer F.Cu) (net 7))
 (segment (start 111.82 86.33) (end 112.111 86.33) (width 0.3) (layer F.Cu) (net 7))
 (segment (start 112.111 86.33) (end 114.9604 89.1794) (width 0.3) (layer F.Cu) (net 7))
 (segment (start 125.3119 92.9613) (end 125.3236 92.973) (width 0.5) (layer F.Cu) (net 9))
 (segment (start 122.8852 92.9613) (end 125.3119 92.9613) (width 0.5) (layer F.Cu) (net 9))
 (segment (start 117.5395 92.973) (end 117.5004 93.0121) (width 0.5) (layer F.Cu) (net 10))
 (segment (start 119.7864 92.973) (end 117.5395 92.973) (width 0.5) (layer F.Cu) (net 10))
 (segment (start 111.465 95.33) (end 111.475 95.32) (width 0.5) (layer F.Cu) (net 11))
 (segment (start 108.62 95.03) (end 111.465 95.03) (width 0.5) (layer F.Cu) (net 11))
 (segment (start 108.6056 95.03) (end 108.62 95.03) (width 0.5) (layer F.Cu) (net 11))
 (segment (start 108.5888 95.0468) (end 108.6056 95.03) (width 0.5) (layer F.Cu) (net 11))
 (segment (start 107.2388 95.0468) (end 108.5888 95.0468) (width 0.5) (layer F.Cu) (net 11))
 (segment (start 108.98 86.33) (end 109.62 86.33) (width 0.5) (layer F.Cu) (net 8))
 (segment (start 108.59 86.33) (end 109.62 86.33) (width 0.5) (layer F.Cu) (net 8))
 (segment (start 105.909999 89.010001) (end 108.59 86.33) (width 0.5) (layer F.Cu) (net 8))
 (segment (start 105.909999 89.100001) (end 105.909999 89.010001) (width 0.5) (layer F.Cu) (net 8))
 (segment (start 105.06 89.95) (end 105.909999 89.100001) (width 0.5) (layer F.Cu) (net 8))
 (segment (start 105.06 89.95) (end 105.06 92.49) (width 0.5) (layer F.Cu) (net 8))
 (segment (start 105.06 92.49) (end 105.06 95.03) (width 0.5) (layer F.Cu) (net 8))
 (segment (start 111.315 92.79) (end 111.495 92.97) (width 0.5) (layer F.Cu) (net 12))
 (segment (start 108.62 92.49) (end 111.315 92.49) (width 0.5) (layer F.Cu) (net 12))
 (segment (start 108.6032 92.5068) (end 107.2388 92.5068) (width 0.5) (layer F.Cu) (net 12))
 (segment (start 108.62 92.49) (end 108.6032 92.5068) (width 0.5) (layer F.Cu) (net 12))
 (segment (start 111.465 90.25) (end 111.475 90.26) (width 0.5) (layer F.Cu) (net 13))
 (segment (start 108.62 89.95) (end 111.465 89.95) (width 0.5) (layer F.Cu) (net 13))
 (segment (start 108.6032 89.9668) (end 107.2388 89.9668) (width 0.5) (layer F.Cu) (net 13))
 (segment (start 108.62 89.95) (end 108.6032 89.9668) (width 0.5) (layer F.Cu) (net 13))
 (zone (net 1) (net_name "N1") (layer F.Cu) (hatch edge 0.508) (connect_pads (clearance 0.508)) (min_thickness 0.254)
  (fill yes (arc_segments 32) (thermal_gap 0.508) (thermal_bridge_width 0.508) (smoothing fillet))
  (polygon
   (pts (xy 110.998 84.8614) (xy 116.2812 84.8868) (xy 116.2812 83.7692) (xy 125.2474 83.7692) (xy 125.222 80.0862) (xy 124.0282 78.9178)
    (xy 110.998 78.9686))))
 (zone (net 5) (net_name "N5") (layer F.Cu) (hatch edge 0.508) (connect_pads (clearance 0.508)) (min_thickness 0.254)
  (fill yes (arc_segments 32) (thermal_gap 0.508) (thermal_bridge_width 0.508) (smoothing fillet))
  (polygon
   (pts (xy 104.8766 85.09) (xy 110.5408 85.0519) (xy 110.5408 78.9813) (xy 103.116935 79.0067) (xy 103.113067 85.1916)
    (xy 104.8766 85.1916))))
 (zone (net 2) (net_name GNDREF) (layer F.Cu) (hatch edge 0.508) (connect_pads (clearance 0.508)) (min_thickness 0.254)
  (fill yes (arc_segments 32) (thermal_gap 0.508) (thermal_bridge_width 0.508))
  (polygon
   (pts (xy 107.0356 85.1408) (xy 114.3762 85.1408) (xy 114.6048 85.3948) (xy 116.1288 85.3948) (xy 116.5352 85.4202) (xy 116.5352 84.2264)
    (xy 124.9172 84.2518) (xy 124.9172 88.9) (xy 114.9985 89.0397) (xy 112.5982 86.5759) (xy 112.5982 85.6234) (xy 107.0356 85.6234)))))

